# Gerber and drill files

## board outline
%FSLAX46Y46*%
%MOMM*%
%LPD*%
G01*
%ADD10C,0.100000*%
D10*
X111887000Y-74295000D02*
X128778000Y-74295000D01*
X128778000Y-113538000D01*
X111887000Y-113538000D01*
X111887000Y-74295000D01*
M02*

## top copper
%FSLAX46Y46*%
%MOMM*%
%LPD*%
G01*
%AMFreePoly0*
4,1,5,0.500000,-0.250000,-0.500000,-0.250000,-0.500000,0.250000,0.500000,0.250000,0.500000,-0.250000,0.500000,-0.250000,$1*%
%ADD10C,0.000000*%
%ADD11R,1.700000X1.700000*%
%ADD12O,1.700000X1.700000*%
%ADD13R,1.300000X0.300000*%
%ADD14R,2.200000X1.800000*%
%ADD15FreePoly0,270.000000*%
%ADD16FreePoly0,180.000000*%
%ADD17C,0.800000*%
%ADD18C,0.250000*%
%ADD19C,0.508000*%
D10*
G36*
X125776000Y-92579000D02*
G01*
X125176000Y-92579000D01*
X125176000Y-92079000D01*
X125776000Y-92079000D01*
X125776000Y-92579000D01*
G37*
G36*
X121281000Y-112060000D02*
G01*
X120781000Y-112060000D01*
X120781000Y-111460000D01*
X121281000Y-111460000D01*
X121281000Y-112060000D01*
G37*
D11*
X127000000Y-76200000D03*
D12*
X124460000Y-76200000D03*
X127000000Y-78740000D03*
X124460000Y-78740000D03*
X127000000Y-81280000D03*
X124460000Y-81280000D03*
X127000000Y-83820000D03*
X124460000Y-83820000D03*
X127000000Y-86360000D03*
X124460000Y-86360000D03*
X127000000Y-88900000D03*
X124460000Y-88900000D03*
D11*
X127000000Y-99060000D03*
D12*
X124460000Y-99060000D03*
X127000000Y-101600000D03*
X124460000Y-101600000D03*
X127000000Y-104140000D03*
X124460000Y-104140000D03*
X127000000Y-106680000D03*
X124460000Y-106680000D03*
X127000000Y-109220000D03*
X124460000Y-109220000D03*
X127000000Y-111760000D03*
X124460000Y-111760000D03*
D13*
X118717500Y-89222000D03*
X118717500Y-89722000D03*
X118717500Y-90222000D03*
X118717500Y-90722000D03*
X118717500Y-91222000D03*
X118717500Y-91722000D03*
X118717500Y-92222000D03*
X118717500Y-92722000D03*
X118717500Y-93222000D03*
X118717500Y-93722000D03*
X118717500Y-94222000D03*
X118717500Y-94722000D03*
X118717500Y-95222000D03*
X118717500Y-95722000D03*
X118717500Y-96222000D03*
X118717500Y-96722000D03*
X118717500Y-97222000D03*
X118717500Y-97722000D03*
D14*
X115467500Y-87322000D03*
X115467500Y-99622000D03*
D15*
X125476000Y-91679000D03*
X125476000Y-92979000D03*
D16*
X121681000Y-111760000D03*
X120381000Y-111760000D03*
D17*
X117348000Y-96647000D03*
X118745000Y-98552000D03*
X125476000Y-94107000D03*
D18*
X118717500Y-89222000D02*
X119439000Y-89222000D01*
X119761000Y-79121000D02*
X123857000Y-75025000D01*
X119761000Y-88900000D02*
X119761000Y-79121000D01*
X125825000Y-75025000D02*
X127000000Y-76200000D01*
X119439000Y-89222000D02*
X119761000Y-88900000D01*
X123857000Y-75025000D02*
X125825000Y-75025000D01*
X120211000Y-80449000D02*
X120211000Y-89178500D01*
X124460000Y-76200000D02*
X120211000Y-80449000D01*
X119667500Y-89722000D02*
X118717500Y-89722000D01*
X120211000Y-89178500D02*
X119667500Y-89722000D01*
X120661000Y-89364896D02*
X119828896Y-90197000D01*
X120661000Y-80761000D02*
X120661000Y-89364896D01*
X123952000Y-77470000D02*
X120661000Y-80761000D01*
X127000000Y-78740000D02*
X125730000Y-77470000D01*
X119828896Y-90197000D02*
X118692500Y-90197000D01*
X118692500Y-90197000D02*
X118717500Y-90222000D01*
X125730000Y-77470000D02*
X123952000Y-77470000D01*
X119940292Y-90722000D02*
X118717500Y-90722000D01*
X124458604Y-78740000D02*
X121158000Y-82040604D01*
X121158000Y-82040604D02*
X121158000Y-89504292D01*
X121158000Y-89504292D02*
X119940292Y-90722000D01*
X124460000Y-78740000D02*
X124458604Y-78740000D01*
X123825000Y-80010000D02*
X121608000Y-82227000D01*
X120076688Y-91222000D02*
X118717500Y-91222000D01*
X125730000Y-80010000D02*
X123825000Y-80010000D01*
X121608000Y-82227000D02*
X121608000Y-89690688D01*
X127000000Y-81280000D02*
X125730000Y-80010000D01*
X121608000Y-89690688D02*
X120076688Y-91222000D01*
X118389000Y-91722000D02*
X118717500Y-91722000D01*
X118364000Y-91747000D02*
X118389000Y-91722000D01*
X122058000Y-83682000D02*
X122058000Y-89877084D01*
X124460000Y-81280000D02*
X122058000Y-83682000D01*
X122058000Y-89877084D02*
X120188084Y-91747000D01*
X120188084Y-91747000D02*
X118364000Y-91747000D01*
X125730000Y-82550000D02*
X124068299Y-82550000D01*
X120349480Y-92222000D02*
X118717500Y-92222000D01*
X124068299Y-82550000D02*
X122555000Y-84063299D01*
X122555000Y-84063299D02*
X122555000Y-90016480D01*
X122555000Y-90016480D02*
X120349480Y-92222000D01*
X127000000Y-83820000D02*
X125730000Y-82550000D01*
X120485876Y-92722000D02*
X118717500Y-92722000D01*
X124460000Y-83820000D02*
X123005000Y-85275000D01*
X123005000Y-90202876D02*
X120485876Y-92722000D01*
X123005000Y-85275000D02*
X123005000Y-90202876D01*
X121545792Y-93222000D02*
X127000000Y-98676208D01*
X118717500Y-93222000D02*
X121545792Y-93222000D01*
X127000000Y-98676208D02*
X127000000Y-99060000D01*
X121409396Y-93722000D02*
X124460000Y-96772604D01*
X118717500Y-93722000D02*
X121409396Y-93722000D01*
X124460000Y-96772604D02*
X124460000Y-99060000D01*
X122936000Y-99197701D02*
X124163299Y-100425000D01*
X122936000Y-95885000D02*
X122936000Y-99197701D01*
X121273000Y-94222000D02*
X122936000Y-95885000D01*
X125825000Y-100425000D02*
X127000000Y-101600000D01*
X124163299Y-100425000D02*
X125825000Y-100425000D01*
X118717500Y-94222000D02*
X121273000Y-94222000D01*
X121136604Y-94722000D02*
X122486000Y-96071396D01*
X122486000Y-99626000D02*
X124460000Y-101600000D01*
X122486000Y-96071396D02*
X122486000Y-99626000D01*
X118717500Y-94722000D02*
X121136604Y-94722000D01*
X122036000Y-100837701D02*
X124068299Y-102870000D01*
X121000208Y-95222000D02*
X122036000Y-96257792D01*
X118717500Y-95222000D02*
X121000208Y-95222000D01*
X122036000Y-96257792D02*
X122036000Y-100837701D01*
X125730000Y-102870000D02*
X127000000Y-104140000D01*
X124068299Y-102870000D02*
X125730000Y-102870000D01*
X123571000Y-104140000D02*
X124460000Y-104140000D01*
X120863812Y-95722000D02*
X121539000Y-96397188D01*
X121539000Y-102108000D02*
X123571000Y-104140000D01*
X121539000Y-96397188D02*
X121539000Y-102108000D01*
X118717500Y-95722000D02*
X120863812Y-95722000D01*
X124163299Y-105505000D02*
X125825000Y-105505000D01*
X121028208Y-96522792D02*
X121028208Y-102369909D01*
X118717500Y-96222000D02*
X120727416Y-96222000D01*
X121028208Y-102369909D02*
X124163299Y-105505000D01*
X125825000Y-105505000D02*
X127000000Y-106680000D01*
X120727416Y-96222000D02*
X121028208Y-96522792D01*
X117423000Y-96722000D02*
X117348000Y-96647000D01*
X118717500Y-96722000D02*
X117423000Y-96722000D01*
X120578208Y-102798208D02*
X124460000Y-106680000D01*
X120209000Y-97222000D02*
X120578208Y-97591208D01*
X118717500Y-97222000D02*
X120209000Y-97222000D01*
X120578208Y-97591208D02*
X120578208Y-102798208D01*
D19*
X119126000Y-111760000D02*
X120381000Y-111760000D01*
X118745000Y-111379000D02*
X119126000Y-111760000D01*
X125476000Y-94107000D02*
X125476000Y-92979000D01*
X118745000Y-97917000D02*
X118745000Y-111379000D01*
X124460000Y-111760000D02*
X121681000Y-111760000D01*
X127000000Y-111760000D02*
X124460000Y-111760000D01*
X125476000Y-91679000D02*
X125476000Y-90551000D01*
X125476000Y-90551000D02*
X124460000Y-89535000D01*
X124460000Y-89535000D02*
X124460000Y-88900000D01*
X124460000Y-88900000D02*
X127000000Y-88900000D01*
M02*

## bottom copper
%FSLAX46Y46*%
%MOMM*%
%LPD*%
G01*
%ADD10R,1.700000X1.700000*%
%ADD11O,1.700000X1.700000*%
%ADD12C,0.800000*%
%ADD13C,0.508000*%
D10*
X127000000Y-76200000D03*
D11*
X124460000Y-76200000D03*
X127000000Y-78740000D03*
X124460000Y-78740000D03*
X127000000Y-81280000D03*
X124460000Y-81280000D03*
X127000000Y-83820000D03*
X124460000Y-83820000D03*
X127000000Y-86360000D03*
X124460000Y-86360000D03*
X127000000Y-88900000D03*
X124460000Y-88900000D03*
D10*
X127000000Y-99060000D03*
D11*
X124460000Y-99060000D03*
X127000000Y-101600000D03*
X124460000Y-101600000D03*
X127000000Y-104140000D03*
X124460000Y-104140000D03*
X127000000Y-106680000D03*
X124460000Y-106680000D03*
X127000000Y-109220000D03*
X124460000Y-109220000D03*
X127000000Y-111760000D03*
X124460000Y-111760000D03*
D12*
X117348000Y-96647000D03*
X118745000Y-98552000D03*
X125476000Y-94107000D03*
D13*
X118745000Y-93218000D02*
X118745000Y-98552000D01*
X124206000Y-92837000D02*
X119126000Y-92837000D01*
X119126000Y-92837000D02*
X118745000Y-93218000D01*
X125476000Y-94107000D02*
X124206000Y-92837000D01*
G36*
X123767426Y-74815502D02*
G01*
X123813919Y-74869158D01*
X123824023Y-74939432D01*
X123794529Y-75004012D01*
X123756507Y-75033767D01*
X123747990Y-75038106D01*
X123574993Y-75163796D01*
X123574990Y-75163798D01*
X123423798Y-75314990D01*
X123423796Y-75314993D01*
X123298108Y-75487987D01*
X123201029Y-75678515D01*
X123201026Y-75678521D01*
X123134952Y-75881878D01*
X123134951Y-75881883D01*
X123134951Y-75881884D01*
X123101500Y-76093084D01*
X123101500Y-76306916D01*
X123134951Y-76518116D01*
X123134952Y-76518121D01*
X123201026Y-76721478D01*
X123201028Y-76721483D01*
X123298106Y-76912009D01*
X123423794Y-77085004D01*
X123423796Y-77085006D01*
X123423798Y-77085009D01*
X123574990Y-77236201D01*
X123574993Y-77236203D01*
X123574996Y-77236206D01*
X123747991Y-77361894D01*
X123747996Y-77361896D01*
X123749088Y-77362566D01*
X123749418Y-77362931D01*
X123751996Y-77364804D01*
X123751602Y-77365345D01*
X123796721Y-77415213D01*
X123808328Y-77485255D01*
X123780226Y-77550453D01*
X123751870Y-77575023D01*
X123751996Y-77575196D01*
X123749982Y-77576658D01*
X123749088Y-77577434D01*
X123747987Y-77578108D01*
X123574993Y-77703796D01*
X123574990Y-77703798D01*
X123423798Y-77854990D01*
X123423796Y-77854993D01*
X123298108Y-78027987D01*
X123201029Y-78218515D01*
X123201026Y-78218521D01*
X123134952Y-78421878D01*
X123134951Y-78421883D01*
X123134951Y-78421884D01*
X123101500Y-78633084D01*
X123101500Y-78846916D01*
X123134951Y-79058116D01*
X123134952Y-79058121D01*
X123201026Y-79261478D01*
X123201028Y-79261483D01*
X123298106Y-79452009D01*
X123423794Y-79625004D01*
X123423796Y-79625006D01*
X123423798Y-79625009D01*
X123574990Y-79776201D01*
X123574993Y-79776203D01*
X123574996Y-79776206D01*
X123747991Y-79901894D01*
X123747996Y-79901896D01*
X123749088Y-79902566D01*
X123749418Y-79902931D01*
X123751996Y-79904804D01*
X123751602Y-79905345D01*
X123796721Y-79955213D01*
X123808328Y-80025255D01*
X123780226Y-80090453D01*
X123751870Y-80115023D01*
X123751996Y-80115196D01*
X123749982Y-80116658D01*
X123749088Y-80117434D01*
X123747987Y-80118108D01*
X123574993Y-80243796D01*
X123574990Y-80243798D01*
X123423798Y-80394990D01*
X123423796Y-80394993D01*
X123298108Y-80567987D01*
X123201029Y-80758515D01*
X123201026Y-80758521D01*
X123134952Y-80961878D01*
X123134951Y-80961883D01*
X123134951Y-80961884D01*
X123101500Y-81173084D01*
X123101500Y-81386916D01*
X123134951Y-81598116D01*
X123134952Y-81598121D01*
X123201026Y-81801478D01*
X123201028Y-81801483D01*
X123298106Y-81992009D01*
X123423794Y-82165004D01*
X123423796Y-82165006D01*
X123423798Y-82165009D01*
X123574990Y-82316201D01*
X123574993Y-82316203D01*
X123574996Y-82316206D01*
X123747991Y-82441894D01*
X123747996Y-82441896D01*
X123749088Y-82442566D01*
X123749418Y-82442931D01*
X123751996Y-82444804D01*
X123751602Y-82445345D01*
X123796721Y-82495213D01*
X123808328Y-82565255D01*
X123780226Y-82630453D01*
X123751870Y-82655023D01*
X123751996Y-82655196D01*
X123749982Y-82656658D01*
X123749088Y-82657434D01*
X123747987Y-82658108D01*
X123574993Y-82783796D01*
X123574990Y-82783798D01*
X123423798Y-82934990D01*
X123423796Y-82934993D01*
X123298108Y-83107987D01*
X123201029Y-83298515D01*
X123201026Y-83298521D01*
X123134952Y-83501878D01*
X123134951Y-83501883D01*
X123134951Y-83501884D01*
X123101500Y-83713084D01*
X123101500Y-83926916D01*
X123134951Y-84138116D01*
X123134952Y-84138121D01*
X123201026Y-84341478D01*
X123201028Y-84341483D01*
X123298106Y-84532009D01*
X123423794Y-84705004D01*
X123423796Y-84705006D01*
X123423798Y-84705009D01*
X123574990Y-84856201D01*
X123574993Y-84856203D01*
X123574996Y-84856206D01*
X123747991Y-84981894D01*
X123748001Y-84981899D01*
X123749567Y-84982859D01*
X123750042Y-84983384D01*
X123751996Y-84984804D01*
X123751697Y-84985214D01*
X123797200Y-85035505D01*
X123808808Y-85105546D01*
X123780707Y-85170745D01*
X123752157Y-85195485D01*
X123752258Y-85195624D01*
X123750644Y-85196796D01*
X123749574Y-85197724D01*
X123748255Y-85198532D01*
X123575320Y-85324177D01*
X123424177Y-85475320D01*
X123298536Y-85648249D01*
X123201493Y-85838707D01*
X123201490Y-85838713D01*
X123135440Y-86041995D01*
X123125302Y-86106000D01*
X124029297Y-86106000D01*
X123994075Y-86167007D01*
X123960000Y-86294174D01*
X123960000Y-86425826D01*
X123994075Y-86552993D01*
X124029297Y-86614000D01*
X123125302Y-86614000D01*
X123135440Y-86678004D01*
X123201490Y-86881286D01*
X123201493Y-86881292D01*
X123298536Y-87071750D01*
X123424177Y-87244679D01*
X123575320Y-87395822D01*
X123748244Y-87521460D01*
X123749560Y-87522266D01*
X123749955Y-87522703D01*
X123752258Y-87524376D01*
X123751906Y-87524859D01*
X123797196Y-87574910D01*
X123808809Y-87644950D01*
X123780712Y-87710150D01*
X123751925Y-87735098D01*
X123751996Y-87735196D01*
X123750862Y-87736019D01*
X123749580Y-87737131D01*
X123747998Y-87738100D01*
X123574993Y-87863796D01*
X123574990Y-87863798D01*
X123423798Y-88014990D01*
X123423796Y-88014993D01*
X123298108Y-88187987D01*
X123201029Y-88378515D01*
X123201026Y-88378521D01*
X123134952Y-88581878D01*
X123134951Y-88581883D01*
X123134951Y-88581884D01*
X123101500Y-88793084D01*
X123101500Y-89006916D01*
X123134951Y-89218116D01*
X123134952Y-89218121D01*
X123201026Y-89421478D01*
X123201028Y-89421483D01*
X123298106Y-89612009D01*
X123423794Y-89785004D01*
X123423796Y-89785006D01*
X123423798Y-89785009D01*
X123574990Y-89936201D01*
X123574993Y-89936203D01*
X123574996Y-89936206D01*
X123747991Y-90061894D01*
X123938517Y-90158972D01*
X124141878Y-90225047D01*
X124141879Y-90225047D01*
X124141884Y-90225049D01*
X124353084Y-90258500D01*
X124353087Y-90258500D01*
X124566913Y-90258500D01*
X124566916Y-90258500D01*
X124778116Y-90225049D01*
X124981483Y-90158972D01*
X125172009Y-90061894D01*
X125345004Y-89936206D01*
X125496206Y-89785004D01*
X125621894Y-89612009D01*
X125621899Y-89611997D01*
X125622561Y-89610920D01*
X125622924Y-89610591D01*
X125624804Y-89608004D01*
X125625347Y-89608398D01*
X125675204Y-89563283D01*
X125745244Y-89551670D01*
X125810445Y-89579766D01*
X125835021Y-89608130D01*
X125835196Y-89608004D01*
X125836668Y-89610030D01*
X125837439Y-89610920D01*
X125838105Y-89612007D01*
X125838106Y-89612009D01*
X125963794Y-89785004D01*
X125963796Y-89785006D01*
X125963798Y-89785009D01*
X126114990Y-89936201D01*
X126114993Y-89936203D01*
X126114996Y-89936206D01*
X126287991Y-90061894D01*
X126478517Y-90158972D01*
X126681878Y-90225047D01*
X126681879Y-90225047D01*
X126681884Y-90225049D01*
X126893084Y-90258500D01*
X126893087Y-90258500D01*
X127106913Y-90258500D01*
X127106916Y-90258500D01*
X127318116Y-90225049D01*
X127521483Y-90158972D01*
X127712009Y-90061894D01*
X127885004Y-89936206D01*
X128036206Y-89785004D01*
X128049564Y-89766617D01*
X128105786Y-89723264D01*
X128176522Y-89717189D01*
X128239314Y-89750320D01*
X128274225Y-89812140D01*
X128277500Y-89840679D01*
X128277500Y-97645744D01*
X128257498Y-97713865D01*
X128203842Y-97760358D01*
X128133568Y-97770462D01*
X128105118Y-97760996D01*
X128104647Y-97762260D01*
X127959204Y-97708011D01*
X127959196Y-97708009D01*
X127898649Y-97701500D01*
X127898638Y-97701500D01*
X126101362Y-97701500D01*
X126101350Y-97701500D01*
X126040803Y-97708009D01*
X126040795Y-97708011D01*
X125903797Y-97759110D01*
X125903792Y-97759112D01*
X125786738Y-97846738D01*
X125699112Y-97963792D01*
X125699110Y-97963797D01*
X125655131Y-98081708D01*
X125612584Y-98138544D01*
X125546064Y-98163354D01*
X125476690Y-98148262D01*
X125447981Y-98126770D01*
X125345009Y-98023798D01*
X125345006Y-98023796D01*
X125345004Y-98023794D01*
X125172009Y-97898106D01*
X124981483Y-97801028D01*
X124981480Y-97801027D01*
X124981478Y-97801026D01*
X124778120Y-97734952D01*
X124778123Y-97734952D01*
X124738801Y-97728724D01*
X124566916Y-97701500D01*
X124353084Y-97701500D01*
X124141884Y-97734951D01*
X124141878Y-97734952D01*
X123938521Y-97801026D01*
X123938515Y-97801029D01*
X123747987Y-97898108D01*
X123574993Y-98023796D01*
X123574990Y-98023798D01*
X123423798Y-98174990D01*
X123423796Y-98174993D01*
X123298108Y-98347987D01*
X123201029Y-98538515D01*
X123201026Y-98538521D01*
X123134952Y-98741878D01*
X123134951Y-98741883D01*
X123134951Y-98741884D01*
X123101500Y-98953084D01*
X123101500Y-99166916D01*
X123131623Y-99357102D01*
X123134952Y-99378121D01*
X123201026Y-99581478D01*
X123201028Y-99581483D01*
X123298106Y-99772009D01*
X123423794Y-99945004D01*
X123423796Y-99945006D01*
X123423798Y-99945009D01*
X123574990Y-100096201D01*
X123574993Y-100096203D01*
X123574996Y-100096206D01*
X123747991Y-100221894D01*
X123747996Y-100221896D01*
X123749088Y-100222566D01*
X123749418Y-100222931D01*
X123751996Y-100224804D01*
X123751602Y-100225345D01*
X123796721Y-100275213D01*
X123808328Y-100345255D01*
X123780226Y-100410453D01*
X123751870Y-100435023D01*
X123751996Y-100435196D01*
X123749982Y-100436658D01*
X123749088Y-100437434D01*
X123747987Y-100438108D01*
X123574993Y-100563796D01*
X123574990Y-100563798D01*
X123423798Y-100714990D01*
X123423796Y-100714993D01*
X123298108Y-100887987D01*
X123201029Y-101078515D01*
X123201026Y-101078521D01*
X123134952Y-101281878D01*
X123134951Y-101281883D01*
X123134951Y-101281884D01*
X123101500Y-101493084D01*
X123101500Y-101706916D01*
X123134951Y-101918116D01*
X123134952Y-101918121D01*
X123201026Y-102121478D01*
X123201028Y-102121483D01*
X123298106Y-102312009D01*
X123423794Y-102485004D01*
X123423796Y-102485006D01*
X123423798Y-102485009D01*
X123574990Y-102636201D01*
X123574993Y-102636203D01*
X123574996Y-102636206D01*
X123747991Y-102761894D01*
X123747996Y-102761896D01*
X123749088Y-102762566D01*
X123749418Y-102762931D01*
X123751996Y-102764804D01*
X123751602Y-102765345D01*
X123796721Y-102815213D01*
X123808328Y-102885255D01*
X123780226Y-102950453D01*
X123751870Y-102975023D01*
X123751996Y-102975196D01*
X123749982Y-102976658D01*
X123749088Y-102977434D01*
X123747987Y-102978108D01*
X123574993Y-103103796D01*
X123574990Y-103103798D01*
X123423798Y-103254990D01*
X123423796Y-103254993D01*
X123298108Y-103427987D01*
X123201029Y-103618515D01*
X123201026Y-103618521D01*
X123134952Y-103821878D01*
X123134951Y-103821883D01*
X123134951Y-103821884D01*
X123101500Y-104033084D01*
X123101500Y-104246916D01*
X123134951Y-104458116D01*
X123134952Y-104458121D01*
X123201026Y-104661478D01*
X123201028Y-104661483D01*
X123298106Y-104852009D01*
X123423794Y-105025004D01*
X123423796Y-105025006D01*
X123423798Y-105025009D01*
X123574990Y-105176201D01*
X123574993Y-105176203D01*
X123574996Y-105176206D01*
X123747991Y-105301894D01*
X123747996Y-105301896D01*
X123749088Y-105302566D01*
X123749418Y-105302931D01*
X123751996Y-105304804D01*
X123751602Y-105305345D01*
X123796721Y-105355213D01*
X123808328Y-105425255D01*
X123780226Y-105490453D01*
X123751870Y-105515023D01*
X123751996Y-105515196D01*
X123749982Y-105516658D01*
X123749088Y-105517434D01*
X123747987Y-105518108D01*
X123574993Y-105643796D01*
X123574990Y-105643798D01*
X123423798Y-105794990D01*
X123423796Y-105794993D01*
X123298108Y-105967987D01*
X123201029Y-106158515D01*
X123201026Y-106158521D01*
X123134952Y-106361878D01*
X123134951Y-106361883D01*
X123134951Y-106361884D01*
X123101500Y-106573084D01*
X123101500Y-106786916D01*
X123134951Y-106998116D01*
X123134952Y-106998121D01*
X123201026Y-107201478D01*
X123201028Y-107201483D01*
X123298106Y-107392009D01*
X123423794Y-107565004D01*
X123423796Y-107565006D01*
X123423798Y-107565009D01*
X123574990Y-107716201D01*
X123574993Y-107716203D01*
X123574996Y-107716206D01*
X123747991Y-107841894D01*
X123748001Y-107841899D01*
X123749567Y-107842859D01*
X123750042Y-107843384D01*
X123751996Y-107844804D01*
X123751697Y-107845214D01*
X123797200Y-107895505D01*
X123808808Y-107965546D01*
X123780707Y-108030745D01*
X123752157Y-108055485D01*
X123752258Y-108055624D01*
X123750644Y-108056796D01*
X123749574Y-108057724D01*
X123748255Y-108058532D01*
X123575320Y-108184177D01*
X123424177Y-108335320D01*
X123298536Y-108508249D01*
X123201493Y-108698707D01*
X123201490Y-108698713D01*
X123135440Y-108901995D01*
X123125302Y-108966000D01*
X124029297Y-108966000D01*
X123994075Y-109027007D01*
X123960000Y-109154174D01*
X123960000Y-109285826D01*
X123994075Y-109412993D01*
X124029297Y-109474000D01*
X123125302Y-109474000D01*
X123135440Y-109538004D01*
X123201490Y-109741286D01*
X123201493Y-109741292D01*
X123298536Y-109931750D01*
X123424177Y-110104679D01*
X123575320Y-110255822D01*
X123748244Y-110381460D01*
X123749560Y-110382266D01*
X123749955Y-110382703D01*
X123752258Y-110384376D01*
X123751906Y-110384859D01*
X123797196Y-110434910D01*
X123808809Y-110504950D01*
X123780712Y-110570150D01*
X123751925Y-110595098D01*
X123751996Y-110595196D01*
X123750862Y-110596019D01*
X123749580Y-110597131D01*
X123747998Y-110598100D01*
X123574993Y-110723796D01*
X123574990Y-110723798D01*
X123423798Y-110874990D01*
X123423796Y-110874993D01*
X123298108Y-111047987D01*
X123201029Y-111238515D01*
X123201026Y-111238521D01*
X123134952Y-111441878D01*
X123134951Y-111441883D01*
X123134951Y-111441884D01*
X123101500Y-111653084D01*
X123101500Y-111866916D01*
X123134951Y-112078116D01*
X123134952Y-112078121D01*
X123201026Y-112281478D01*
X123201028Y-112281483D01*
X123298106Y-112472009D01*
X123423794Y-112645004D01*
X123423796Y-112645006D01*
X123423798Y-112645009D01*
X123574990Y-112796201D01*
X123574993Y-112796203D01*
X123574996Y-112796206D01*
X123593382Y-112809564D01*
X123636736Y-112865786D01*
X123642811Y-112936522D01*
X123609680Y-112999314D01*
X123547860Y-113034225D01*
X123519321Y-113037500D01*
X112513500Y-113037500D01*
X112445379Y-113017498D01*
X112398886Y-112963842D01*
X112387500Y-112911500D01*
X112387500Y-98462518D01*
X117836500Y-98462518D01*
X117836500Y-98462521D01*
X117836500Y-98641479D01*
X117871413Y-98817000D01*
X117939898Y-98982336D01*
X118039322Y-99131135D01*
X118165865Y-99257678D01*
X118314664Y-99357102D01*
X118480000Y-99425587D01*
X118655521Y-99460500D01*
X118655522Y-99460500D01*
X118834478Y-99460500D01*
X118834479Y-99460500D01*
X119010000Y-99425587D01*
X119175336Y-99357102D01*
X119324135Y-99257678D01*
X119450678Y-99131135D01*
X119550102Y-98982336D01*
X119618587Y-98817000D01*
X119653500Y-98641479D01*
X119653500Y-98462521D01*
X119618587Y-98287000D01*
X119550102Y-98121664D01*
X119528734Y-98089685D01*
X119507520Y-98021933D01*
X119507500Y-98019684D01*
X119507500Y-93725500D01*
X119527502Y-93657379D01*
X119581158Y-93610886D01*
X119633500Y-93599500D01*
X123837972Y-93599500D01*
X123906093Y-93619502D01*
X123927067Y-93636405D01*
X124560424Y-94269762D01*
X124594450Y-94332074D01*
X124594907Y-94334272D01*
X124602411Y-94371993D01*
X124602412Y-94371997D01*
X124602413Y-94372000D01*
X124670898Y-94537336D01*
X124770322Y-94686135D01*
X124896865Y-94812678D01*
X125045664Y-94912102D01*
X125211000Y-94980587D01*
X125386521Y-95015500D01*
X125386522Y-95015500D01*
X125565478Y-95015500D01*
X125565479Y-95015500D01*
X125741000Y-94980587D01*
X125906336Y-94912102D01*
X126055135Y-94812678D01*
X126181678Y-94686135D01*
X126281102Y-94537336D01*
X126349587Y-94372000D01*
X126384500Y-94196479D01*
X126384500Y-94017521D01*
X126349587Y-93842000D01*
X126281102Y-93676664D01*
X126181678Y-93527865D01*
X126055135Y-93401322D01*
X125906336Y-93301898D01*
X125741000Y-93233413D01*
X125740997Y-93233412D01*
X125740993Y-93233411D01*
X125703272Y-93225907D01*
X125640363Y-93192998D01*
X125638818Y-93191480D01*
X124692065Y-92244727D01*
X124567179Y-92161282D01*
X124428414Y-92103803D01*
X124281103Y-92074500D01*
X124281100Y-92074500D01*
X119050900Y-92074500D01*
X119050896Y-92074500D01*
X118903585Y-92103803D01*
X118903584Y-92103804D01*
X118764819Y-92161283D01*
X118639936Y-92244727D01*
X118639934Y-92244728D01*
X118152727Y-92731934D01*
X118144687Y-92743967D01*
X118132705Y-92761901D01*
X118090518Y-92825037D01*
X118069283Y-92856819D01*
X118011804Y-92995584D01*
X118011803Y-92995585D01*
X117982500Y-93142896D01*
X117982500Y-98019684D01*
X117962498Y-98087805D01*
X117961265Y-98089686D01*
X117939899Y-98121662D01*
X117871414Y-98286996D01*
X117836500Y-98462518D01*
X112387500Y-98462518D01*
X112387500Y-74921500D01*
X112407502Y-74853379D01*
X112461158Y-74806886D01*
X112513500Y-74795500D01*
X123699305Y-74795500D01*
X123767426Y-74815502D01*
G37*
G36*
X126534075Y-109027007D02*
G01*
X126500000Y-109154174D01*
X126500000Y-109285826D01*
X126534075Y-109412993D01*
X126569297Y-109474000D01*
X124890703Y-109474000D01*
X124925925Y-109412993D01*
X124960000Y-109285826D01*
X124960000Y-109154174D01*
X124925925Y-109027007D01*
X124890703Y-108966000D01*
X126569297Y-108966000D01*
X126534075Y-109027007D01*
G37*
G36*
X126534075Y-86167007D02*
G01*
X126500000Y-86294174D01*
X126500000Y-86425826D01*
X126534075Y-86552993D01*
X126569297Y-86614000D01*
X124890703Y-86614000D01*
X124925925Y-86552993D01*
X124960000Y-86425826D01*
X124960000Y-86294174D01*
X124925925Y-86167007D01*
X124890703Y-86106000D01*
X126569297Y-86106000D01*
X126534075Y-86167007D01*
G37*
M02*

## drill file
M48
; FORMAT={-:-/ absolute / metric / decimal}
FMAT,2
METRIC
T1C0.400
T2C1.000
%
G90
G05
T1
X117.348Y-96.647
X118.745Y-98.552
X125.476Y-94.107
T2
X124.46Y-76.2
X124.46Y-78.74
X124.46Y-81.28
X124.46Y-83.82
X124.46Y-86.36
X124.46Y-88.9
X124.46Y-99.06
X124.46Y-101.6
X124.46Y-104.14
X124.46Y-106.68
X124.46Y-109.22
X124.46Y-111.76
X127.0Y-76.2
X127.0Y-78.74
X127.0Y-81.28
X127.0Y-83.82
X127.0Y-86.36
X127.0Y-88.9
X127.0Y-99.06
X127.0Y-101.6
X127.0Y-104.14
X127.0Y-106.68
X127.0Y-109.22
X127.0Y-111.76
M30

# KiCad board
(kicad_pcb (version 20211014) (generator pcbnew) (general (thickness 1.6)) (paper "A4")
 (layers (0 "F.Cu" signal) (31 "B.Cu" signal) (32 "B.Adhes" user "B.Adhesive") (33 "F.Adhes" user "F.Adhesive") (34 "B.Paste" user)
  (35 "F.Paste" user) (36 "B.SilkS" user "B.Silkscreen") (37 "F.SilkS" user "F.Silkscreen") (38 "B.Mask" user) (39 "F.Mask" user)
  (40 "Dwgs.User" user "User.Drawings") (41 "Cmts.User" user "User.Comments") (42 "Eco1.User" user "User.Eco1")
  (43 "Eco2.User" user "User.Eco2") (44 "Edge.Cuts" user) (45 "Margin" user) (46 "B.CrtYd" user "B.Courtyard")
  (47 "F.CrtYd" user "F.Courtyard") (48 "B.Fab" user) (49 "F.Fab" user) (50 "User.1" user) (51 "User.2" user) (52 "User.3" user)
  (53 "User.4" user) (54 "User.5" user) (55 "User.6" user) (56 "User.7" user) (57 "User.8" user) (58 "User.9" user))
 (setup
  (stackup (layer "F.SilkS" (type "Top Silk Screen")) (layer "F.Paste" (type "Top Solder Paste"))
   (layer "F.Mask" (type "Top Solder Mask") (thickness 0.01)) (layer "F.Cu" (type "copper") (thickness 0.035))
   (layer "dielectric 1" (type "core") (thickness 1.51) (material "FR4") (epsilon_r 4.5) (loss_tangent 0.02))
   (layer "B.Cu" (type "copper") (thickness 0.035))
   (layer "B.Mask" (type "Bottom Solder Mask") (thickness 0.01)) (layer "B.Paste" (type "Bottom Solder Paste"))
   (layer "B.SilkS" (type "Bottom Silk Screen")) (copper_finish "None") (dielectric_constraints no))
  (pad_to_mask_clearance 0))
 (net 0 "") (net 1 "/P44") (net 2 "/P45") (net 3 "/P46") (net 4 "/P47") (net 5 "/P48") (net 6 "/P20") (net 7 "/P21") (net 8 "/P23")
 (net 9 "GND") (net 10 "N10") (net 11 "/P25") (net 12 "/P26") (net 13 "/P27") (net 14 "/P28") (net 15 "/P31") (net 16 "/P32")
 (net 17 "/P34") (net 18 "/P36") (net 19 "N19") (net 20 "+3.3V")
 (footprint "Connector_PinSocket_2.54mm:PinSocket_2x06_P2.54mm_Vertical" (layer "F.Cu") (at 127 76.2)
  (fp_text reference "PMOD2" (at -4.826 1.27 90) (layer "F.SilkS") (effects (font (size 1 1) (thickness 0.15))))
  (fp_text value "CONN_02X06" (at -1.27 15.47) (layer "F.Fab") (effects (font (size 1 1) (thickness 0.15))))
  (pad "1" thru_hole rect (at 0 0) (size 1.7 1.7) (drill 1) (layers *.Cu *.Mask) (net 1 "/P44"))
  (pad "2" thru_hole oval (at -2.54 0) (size 1.7 1.7) (drill 1) (layers *.Cu *.Mask) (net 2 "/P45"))
  (pad "3" thru_hole oval (at 0 2.54) (size 1.7 1.7) (drill 1) (layers *.Cu *.Mask) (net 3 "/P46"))
  (pad "4" thru_hole oval (at -2.54 2.54) (size 1.7 1.7) (drill 1) (layers *.Cu *.Mask) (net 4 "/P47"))
  (pad "5" thru_hole oval (at 0 5.08) (size 1.7 1.7) (drill 1) (layers *.Cu *.Mask) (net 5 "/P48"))
  (pad "6" thru_hole oval (at -2.54 5.08) (size 1.7 1.7) (drill 1) (layers *.Cu *.Mask) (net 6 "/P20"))
  (pad "7" thru_hole oval (at 0 7.62) (size 1.7 1.7) (drill 1) (layers *.Cu *.Mask) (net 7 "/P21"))
  (pad "8" thru_hole oval (at -2.54 7.62) (size 1.7 1.7) (drill 1) (layers *.Cu *.Mask) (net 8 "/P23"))
  (pad "9" thru_hole oval (at 0 10.16) (size 1.7 1.7) (drill 1) (layers *.Cu *.Mask) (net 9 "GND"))
  (pad "10" thru_hole oval (at -2.54 10.16) (size 1.7 1.7) (drill 1) (layers *.Cu *.Mask) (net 9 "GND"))
  (pad "11" thru_hole oval (at 0 12.7) (size 1.7 1.7) (drill 1) (layers *.Cu *.Mask) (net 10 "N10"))
  (pad "12" thru_hole oval (at -2.54 12.7) (size 1.7 1.7) (drill 1) (layers *.Cu *.Mask) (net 10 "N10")))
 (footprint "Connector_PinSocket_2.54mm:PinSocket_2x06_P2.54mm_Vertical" (layer "F.Cu") (at 127 99.06)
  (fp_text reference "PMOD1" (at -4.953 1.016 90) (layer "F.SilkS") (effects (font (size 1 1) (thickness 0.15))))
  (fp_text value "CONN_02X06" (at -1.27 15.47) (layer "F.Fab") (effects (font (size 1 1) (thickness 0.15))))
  (pad "1" thru_hole rect (at 0 0) (size 1.7 1.7) (drill 1) (layers *.Cu *.Mask) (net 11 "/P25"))
  (pad "2" thru_hole oval (at -2.54 0) (size 1.7 1.7) (drill 1) (layers *.Cu *.Mask) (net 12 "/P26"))
  (pad "3" thru_hole oval (at 0 2.54) (size 1.7 1.7) (drill 1) (layers *.Cu *.Mask) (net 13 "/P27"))
  (pad "4" thru_hole oval (at -2.54 2.54) (size 1.7 1.7) (drill 1) (layers *.Cu *.Mask) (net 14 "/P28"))
  (pad "5" thru_hole oval (at 0 5.08) (size 1.7 1.7) (drill 1) (layers *.Cu *.Mask) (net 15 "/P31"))
  (pad "6" thru_hole oval (at -2.54 5.08) (size 1.7 1.7) (drill 1) (layers *.Cu *.Mask) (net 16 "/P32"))
  (pad "7" thru_hole oval (at 0 7.62) (size 1.7 1.7) (drill 1) (layers *.Cu *.Mask) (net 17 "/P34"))
  (pad "8" thru_hole oval (at -2.54 7.62) (size 1.7 1.7) (drill 1) (layers *.Cu *.Mask) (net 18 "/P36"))
  (pad "9" thru_hole oval (at 0 10.16) (size 1.7 1.7) (drill 1) (layers *.Cu *.Mask) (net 9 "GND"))
  (pad "10" thru_hole oval (at -2.54 10.16) (size 1.7 1.7) (drill 1) (layers *.Cu *.Mask) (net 9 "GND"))
  (pad "11" thru_hole oval (at 0 12.7) (size 1.7 1.7) (drill 1) (layers *.Cu *.Mask) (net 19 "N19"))
  (pad "12" thru_hole oval (at -2.54 12.7) (size 1.7 1.7) (drill 1) (layers *.Cu *.Mask) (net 19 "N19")))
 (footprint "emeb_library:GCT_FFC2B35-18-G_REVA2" (layer "F.Cu") (at 115.4675 93.472 -90)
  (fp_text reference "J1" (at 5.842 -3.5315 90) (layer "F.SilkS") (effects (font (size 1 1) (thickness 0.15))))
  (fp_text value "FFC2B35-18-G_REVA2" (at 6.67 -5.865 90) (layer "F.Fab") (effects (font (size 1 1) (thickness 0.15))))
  (pad "1" smd rect locked (at -4.25 -3.25 270) (size 0.3 1.3) (layers "F.Cu" "F.Paste" "F.Mask") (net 1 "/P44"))
  (pad "2" smd rect locked (at -3.75 -3.25 270) (size 0.3 1.3) (layers "F.Cu" "F.Paste" "F.Mask") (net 2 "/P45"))
  (pad "3" smd rect locked (at -3.25 -3.25 270) (size 0.3 1.3) (layers "F.Cu" "F.Paste" "F.Mask") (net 3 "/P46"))
  (pad "4" smd rect locked (at -2.75 -3.25 270) (size 0.3 1.3) (layers "F.Cu" "F.Paste" "F.Mask") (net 4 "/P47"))
  (pad "5" smd rect locked (at -2.25 -3.25 270) (size 0.3 1.3) (layers "F.Cu" "F.Paste" "F.Mask") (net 5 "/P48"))
  (pad "6" smd rect locked (at -1.75 -3.25 270) (size 0.3 1.3) (layers "F.Cu" "F.Paste" "F.Mask") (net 6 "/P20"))
  (pad "7" smd rect locked (at -1.25 -3.25 270) (size 0.3 1.3) (layers "F.Cu" "F.Paste" "F.Mask") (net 7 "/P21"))
  (pad "8" smd rect locked (at -0.75 -3.25 270) (size 0.3 1.3) (layers "F.Cu" "F.Paste" "F.Mask") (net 8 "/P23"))
  (pad "9" smd rect locked (at -0.25 -3.25 270) (size 0.3 1.3) (layers "F.Cu" "F.Paste" "F.Mask") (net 11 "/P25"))
  (pad "10" smd rect locked (at 0.25 -3.25 270) (size 0.3 1.3) (layers "F.Cu" "F.Paste" "F.Mask") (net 12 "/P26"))
  (pad "11" smd rect locked (at 0.75 -3.25 270) (size 0.3 1.3) (layers "F.Cu" "F.Paste" "F.Mask") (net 13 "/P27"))
  (pad "12" smd rect locked (at 1.25 -3.25 270) (size 0.3 1.3) (layers "F.Cu" "F.Paste" "F.Mask") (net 14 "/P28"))
  (pad "13" smd rect locked (at 1.75 -3.25 270) (size 0.3 1.3) (layers "F.Cu" "F.Paste" "F.Mask") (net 15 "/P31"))
  (pad "14" smd rect locked (at 2.25 -3.25 270) (size 0.3 1.3) (layers "F.Cu" "F.Paste" "F.Mask") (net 16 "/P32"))
  (pad "15" smd rect locked (at 2.75 -3.25 270) (size 0.3 1.3) (layers "F.Cu" "F.Paste" "F.Mask") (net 17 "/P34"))
  (pad "16" smd rect locked (at 3.25 -3.25 270) (size 0.3 1.3) (layers "F.Cu" "F.Paste" "F.Mask") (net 9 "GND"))
  (pad "17" smd rect locked (at 3.75 -3.25 270) (size 0.3 1.3) (layers "F.Cu" "F.Paste" "F.Mask") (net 18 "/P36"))
  (pad "18" smd rect locked (at 4.25 -3.25 270) (size 0.3 1.3) (layers "F.Cu" "F.Paste" "F.Mask") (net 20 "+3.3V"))
  (pad "S1" smd rect locked (at -6.15 0 270) (size 1.8 2.2) (layers "F.Cu" "F.Paste" "F.Mask"))
  (pad "S2" smd rect locked (at 6.15 0 270) (size 1.8 2.2) (layers "F.Cu" "F.Paste" "F.Mask")))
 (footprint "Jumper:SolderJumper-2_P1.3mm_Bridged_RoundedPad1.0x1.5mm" (layer "F.Cu") (at 125.476 92.329 -90)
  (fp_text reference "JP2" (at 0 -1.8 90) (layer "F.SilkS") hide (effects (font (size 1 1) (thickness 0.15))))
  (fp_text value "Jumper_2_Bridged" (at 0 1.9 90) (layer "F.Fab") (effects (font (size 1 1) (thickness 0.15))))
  (fp_poly (pts (xy 0.25 -0.3) (xy -0.25 -0.3) (xy -0.25 0.3) (xy 0.25 0.3)) (layer "F.Cu") (width 0) (fill solid))
  (pad "1" smd custom (at -0.65 0 270) (size 1 0.5) (layers "F.Cu" "F.Mask") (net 10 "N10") (zone_connect 2)
   (options (clearance outline) (anchor rect)) (primitives))
  (pad "2" smd custom (at 0.65 0 270) (size 1 0.5) (layers "F.Cu" "F.Mask") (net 20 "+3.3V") (zone_connect 2)
   (options (clearance outline) (anchor rect)) (primitives)))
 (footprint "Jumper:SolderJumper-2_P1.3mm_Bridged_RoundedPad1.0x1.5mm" (layer "F.Cu") (at 121.031 111.76 180)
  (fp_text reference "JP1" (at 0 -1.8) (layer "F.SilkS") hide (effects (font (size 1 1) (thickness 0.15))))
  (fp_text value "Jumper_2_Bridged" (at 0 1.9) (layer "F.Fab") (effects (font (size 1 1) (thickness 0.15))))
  (fp_poly (pts (xy 0.25 -0.3) (xy -0.25 -0.3) (xy -0.25 0.3) (xy 0.25 0.3)) (layer "F.Cu") (width 0) (fill solid))
  (pad "1" smd custom (at -0.65 0 180) (size 1 0.5) (layers "F.Cu" "F.Mask") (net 19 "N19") (zone_connect 2)
   (options (clearance outline) (anchor rect)) (primitives))
  (pad "2" smd custom (at 0.65 0 180) (size 1 0.5) (layers "F.Cu" "F.Mask") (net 20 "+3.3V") (zone_connect 2)
   (options (clearance outline) (anchor rect)) (primitives)))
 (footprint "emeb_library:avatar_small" (layer "B.Cu") (at 119.761 92.329 90)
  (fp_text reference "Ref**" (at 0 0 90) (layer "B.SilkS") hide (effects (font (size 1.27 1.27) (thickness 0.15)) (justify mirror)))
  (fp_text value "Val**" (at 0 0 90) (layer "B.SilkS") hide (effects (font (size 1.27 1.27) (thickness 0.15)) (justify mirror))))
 (gr_rect (start 128.778 74.295) (end 111.887 113.538) (layer "Edge.Cuts") (width 0.1) (fill none))
 (segment (start 118.7175 89.222) (end 119.439 89.222) (width 0.25) (layer "F.Cu") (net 1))
 (segment (start 119.761 79.121) (end 123.857 75.025) (width 0.25) (layer "F.Cu") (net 1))
 (segment (start 119.761 88.9) (end 119.761 79.121) (width 0.25) (layer "F.Cu") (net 1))
 (segment (start 125.825 75.025) (end 127 76.2) (width 0.25) (layer "F.Cu") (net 1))
 (segment (start 119.439 89.222) (end 119.761 88.9) (width 0.25) (layer "F.Cu") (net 1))
 (segment (start 123.857 75.025) (end 125.825 75.025) (width 0.25) (layer "F.Cu") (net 1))
 (segment (start 120.211 80.449) (end 120.211 89.1785) (width 0.25) (layer "F.Cu") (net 2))
 (segment (start 124.46 76.2) (end 120.211 80.449) (width 0.25) (layer "F.Cu") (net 2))
 (segment (start 119.6675 89.722) (end 118.7175 89.722) (width 0.25) (layer "F.Cu") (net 2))
 (segment (start 120.211 89.1785) (end 119.6675 89.722) (width 0.25) (layer "F.Cu") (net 2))
 (segment (start 120.661 89.364896) (end 119.828896 90.197) (width 0.25) (layer "F.Cu") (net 3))
 (segment (start 120.661 80.761) (end 120.661 89.364896) (width 0.25) (layer "F.Cu") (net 3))
 (segment (start 123.952 77.47) (end 120.661 80.761) (width 0.25) (layer "F.Cu") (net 3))
 (segment (start 127 78.74) (end 125.73 77.47) (width 0.25) (layer "F.Cu") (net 3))
 (segment (start 119.828896 90.197) (end 118.6925 90.197) (width 0.25) (layer "F.Cu") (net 3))
 (segment (start 118.6925 90.197) (end 118.7175 90.222) (width 0.25) (layer "F.Cu") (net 3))
 (segment (start 125.73 77.47) (end 123.952 77.47) (width 0.25) (layer "F.Cu") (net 3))
 (segment (start 119.940292 90.722) (end 118.7175 90.722) (width 0.25) (layer "F.Cu") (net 4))
 (segment (start 124.458604 78.74) (end 121.158 82.040604) (width 0.25) (layer "F.Cu") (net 4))
 (segment (start 121.158 82.040604) (end 121.158 89.504292) (width 0.25) (layer "F.Cu") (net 4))
 (segment (start 121.158 89.504292) (end 119.940292 90.722) (width 0.25) (layer "F.Cu") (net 4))
 (segment (start 124.46 78.74) (end 124.458604 78.74) (width 0.25) (layer "F.Cu") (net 4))
 (segment (start 123.825 80.01) (end 121.608 82.227) (width 0.25) (layer "F.Cu") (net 5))
 (segment (start 120.076688 91.222) (end 118.7175 91.222) (width 0.25) (layer "F.Cu") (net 5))
 (segment (start 125.73 80.01) (end 123.825 80.01) (width 0.25) (layer "F.Cu") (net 5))
 (segment (start 121.608 82.227) (end 121.608 89.690688) (width 0.25) (layer "F.Cu") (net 5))
 (segment (start 127 81.28) (end 125.73 80.01) (width 0.25) (layer "F.Cu") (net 5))
 (segment (start 121.608 89.690688) (end 120.076688 91.222) (width 0.25) (layer "F.Cu") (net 5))
 (segment (start 118.389 91.722) (end 118.7175 91.722) (width 0.25) (layer "F.Cu") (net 6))
 (segment (start 118.364 91.747) (end 118.389 91.722) (width 0.25) (layer "F.Cu") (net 6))
 (segment (start 122.058 83.682) (end 122.058 89.877084) (width 0.25) (layer "F.Cu") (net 6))
 (segment (start 124.46 81.28) (end 122.058 83.682) (width 0.25) (layer "F.Cu") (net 6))
 (segment (start 122.058 89.877084) (end 120.188084 91.747) (width 0.25) (layer "F.Cu") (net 6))
 (segment (start 120.188084 91.747) (end 118.364 91.747) (width 0.25) (layer "F.Cu") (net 6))
 (segment (start 125.73 82.55) (end 124.068299 82.55) (width 0.25) (layer "F.Cu") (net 7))
 (segment (start 120.34948 92.222) (end 118.7175 92.222) (width 0.25) (layer "F.Cu") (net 7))
 (segment (start 124.068299 82.55) (end 122.555 84.063299) (width 0.25) (layer "F.Cu") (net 7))
 (segment (start 122.555 84.063299) (end 122.555 90.01648) (width 0.25) (layer "F.Cu") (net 7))
 (segment (start 122.555 90.01648) (end 120.34948 92.222) (width 0.25) (layer "F.Cu") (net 7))
 (segment (start 127 83.82) (end 125.73 82.55) (width 0.25) (layer "F.Cu") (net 7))
 (segment (start 120.485876 92.722) (end 118.7175 92.722) (width 0.25) (layer "F.Cu") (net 8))
 (segment (start 124.46 83.82) (end 123.005 85.275) (width 0.25) (layer "F.Cu") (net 8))
 (segment (start 123.005 90.202876) (end 120.485876 92.722) (width 0.25) (layer "F.Cu") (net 8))
 (segment (start 123.005 85.275) (end 123.005 90.202876) (width 0.25) (layer "F.Cu") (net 8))
 (segment (start 121.545792 93.222) (end 127 98.676208) (width 0.25) (layer "F.Cu") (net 11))
 (segment (start 118.7175 93.222) (end 121.545792 93.222) (width 0.25) (layer "F.Cu") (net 11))
 (segment (start 127 98.676208) (end 127 99.06) (width 0.25) (layer "F.Cu") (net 11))
 (segment (start 121.409396 93.722) (end 124.46 96.772604) (width 0.25) (layer "F.Cu") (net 12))
 (segment (start 118.7175 93.722) (end 121.409396 93.722) (width 0.25) (layer "F.Cu") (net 12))
 (segment (start 124.46 96.772604) (end 124.46 99.06) (width 0.25) (layer "F.Cu") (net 12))
 (segment (start 122.936 99.197701) (end 124.163299 100.425) (width 0.25) (layer "F.Cu") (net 13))
 (segment (start 122.936 95.885) (end 122.936 99.197701) (width 0.25) (layer "F.Cu") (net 13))
 (segment (start 121.273 94.222) (end 122.936 95.885) (width 0.25) (layer "F.Cu") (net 13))
 (segment (start 125.825 100.425) (end 127 101.6) (width 0.25) (layer "F.Cu") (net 13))
 (segment (start 124.163299 100.425) (end 125.825 100.425) (width 0.25) (layer "F.Cu") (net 13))
 (segment (start 118.7175 94.222) (end 121.273 94.222) (width 0.25) (layer "F.Cu") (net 13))
 (segment (start 121.136604 94.722) (end 122.486 96.071396) (width 0.25) (layer "F.Cu") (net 14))
 (segment (start 122.486 99.626) (end 124.46 101.6) (width 0.25) (layer "F.Cu") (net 14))
 (segment (start 122.486 96.071396) (end 122.486 99.626) (width 0.25) (layer "F.Cu") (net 14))
 (segment (start 118.7175 94.722) (end 121.136604 94.722) (width 0.25) (layer "F.Cu") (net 14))
 (segment (start 122.036 100.837701) (end 124.068299 102.87) (width 0.25) (layer "F.Cu") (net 15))
 (segment (start 121.000208 95.222) (end 122.036 96.257792) (width 0.25) (layer "F.Cu") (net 15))
 (segment (start 118.7175 95.222) (end 121.000208 95.222) (width 0.25) (layer "F.Cu") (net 15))
 (segment (start 122.036 96.257792) (end 122.036 100.837701) (width 0.25) (layer "F.Cu") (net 15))
 (segment (start 125.73 102.87) (end 127 104.14) (width 0.25) (layer "F.Cu") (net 15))
 (segment (start 124.068299 102.87) (end 125.73 102.87) (width 0.25) (layer "F.Cu") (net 15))
 (segment (start 123.571 104.14) (end 124.46 104.14) (width 0.25) (layer "F.Cu") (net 16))
 (segment (start 120.863812 95.722) (end 121.539 96.397188) (width 0.25) (layer "F.Cu") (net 16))
 (segment (start 121.539 102.108) (end 123.571 104.14) (width 0.25) (layer "F.Cu") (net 16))
 (segment (start 121.539 96.397188) (end 121.539 102.108) (width 0.25) (layer "F.Cu") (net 16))
 (segment (start 118.7175 95.722) (end 120.863812 95.722) (width 0.25) (layer "F.Cu") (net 16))
 (segment (start 124.163299 105.505) (end 125.825 105.505) (width 0.25) (layer "F.Cu") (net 17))
 (segment (start 121.028208 96.522792) (end 121.028208 102.369909) (width 0.25) (layer "F.Cu") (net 17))
 (segment (start 118.7175 96.222) (end 120.727416 96.222) (width 0.25) (layer "F.Cu") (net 17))
 (segment (start 121.028208 102.369909) (end 124.163299 105.505) (width 0.25) (layer "F.Cu") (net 17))
 (segment (start 125.825 105.505) (end 127 106.68) (width 0.25) (layer "F.Cu") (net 17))
 (segment (start 120.727416 96.222) (end 121.028208 96.522792) (width 0.25) (layer "F.Cu") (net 17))
 (segment (start 117.423 96.722) (end 117.348 96.647) (width 0.25) (layer "F.Cu") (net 9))
 (segment (start 118.7175 96.722) (end 117.423 96.722) (width 0.25) (layer "F.Cu") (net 9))
 (via (at 117.348 96.647) (size 0.8) (drill 0.4) (layers "F.Cu" "B.Cu") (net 9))
 (segment (start 120.578208 102.798208) (end 124.46 106.68) (width 0.25) (layer "F.Cu") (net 18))
 (segment (start 120.209 97.222) (end 120.578208 97.591208) (width 0.25) (layer "F.Cu") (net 18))
 (segment (start 118.7175 97.222) (end 120.209 97.222) (width 0.25) (layer "F.Cu") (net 18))
 (segment (start 120.578208 97.591208) (end 120.578208 102.798208) (width 0.25) (layer "F.Cu") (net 18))
 (segment (start 119.126 111.76) (end 120.381 111.76) (width 0.508) (layer "F.Cu") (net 20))
 (segment (start 118.745 111.379) (end 119.126 111.76) (width 0.508) (layer "F.Cu") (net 20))
 (segment (start 125.476 94.107) (end 125.476 92.979) (width 0.508) (layer "F.Cu") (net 20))
 (segment (start 118.745 97.917) (end 118.745 111.379) (width 0.508) (layer "F.Cu") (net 20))
 (via (at 118.745 98.552) (size 0.8) (drill 0.4) (layers "F.Cu" "B.Cu") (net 20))
 (via (at 125.476 94.107) (size 0.8) (drill 0.4) (layers "F.Cu" "B.Cu") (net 20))
 (segment (start 118.745 93.218) (end 118.745 98.552) (width 0.508) (layer "B.Cu") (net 20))
 (segment (start 124.206 92.837) (end 119.126 92.837) (width 0.508) (layer "B.Cu") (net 20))
 (segment (start 119.126 92.837) (end 118.745 93.218) (width 0.508) (layer "B.Cu") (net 20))
 (segment (start 125.476 94.107) (end 124.206 92.837) (width 0.508) (layer "B.Cu") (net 20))
 (segment (start 124.46 111.76) (end 121.681 111.76) (width 0.508) (layer "F.Cu") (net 19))
 (segment (start 127 111.76) (end 124.46 111.76) (width 0.508) (layer "F.Cu") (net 19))
 (segment (start 125.476 91.679) (end 125.476 90.551) (width 0.508) (layer "F.Cu") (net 10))
 (segment (start 125.476 90.551) (end 124.46 89.535) (width 0.508) (layer "F.Cu") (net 10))
 (segment (start 124.46 89.535) (end 124.46 88.9) (width 0.508) (layer "F.Cu") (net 10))
 (segment (start 124.46 88.9) (end 127 88.9) (width 0.508) (layer "F.Cu") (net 10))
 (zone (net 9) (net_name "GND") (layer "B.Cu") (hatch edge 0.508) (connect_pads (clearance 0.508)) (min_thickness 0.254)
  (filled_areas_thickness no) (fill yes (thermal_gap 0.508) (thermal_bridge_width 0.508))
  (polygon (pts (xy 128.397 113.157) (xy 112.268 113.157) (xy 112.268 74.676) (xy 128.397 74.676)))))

